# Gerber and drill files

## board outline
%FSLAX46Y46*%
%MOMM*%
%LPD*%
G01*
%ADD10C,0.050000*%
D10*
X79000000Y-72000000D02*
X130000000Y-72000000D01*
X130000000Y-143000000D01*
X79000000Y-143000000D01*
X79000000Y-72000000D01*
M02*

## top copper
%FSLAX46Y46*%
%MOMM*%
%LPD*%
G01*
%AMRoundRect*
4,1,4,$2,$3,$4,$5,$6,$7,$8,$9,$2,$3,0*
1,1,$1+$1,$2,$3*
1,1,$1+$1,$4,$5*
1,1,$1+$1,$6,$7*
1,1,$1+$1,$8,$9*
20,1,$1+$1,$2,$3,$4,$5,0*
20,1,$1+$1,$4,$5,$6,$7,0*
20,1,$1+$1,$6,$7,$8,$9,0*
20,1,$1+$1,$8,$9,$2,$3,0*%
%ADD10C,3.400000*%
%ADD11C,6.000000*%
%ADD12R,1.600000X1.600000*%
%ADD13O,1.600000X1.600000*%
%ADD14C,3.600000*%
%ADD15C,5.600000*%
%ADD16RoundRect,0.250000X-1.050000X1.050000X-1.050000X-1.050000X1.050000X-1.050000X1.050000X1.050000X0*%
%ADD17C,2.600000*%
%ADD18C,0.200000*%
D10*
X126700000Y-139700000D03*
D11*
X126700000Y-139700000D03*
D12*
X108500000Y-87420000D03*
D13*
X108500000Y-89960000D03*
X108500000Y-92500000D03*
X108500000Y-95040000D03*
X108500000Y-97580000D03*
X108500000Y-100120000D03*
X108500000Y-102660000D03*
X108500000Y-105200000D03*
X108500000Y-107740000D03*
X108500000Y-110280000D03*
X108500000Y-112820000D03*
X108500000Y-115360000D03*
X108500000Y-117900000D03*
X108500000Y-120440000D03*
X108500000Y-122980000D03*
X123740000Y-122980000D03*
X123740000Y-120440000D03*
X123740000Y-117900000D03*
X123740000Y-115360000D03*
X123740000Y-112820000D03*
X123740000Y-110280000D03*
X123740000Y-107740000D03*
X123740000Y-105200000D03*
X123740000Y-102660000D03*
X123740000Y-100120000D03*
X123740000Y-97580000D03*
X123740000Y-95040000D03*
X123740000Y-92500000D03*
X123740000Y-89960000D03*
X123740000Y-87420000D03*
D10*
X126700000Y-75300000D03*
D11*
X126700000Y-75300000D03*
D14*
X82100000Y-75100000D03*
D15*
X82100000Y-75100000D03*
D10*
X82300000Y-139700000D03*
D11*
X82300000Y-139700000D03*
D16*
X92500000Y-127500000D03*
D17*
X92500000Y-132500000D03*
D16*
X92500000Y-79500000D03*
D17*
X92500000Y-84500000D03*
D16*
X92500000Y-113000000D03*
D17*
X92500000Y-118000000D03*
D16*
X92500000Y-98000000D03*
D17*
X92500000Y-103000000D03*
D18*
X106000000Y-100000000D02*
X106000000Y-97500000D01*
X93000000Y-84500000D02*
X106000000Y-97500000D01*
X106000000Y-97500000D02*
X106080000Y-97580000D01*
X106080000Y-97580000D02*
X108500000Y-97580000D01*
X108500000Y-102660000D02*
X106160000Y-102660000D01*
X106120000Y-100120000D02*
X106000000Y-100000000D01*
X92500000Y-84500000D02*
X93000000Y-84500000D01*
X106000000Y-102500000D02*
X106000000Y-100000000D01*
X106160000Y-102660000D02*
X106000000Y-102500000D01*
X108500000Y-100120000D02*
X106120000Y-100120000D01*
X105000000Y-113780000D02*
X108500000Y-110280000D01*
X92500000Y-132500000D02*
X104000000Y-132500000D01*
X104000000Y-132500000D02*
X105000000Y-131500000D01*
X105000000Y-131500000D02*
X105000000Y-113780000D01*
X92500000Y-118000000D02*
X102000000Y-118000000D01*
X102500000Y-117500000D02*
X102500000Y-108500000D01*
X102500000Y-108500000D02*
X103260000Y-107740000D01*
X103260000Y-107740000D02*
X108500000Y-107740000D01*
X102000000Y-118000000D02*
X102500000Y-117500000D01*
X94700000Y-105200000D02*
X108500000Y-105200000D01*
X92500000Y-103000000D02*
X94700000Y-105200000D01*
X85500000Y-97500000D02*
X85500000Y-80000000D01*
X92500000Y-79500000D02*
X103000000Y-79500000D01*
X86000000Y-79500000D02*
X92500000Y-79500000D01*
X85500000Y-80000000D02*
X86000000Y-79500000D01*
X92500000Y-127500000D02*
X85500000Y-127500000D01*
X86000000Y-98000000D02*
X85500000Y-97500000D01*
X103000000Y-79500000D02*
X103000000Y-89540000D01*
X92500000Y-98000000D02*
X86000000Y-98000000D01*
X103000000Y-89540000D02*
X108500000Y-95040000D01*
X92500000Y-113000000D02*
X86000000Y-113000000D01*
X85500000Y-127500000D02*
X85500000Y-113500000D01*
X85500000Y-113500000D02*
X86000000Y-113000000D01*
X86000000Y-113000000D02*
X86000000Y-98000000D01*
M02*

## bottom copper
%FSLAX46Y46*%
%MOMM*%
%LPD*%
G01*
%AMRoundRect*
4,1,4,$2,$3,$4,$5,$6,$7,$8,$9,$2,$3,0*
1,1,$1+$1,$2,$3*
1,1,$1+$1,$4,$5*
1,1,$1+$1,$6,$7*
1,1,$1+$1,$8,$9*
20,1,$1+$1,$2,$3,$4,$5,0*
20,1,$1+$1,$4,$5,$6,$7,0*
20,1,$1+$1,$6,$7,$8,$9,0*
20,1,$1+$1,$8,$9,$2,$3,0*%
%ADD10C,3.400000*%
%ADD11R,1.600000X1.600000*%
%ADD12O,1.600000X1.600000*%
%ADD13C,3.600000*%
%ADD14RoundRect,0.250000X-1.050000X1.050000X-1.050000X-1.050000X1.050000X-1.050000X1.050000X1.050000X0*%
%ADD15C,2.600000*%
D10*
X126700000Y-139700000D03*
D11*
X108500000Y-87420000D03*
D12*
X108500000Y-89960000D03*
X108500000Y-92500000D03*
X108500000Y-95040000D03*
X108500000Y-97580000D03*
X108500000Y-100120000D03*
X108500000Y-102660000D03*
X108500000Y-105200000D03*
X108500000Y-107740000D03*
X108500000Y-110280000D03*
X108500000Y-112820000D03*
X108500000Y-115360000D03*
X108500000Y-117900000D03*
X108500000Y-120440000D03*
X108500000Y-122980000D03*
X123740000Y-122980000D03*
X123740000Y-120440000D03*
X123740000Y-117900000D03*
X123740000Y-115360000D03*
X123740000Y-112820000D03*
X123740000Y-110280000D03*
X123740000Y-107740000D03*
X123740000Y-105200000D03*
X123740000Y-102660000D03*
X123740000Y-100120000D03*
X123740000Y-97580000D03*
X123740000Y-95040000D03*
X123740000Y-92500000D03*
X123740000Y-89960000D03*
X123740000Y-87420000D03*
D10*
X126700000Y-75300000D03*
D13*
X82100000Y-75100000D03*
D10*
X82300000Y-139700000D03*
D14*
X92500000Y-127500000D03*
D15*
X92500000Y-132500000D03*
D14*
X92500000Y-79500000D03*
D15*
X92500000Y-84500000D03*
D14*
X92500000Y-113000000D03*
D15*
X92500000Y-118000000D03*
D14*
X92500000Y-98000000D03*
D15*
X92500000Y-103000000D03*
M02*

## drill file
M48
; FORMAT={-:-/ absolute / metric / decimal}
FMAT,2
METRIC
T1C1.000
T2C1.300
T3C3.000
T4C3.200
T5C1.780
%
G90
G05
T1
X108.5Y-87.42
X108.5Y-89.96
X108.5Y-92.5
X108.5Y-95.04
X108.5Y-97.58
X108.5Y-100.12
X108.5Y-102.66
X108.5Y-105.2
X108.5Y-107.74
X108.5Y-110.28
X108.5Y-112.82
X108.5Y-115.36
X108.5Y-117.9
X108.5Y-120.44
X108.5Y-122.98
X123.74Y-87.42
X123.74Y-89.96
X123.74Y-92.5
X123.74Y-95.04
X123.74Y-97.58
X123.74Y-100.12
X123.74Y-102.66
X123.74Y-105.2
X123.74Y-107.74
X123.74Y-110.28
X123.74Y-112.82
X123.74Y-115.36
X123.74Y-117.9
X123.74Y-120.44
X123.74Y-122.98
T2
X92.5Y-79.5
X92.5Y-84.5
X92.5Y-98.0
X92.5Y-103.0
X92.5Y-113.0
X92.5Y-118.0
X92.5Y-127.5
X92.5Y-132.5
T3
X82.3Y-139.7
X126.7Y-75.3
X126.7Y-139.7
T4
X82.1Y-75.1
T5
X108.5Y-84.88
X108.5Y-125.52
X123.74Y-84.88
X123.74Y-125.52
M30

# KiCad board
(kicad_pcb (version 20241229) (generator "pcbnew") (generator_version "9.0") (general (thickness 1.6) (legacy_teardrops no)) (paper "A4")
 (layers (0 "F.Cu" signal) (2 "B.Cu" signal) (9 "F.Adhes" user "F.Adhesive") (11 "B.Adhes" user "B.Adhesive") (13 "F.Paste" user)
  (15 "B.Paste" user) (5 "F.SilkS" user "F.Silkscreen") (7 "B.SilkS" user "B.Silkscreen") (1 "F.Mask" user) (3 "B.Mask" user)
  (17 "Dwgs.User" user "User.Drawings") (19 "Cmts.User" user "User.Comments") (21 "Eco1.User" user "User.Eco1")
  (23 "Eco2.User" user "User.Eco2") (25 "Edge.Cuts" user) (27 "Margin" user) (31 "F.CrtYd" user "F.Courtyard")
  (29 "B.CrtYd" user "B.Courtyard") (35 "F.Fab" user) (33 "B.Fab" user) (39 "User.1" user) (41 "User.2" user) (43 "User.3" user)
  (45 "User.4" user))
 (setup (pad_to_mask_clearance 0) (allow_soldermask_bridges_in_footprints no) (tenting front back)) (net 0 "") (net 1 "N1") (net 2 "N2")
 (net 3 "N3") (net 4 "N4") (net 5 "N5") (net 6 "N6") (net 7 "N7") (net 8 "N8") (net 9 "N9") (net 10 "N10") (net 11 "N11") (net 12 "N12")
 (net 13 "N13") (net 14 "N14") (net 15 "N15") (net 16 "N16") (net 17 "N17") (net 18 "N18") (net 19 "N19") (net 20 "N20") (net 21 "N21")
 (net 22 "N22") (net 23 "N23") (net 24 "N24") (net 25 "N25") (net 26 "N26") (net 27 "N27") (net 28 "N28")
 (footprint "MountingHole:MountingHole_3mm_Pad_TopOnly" (layer "F.Cu") (at 126.7 139.7)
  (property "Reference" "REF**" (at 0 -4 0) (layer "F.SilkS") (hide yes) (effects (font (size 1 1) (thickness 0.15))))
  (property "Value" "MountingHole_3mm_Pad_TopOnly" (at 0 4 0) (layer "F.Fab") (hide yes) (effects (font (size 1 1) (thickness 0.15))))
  (pad "1" thru_hole circle (at 0 0) (size 3.4 3.4) (drill 3) (layers "*.Cu" "*.Mask") (remove_unused_layers no))
  (pad "1" connect circle (at 0 0) (size 6 6) (layers "F.Cu" "F.Mask")))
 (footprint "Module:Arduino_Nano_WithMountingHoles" (layer "F.Cu") (at 108.5 87.42)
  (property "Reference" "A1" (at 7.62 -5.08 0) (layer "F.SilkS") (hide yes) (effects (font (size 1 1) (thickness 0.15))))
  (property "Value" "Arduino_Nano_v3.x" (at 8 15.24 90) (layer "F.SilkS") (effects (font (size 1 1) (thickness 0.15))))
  (pad "" np_thru_hole circle (at 0 -2.54) (size 1.78 1.78) (drill 1.78) (layers "*.Cu" "*.Mask"))
  (pad "" np_thru_hole circle (at 0 38.1) (size 1.78 1.78) (drill 1.78) (layers "*.Cu" "*.Mask"))
  (pad "" np_thru_hole circle (at 15.24 -2.54) (size 1.78 1.78) (drill 1.78) (layers "*.Cu" "*.Mask"))
  (pad "" np_thru_hole circle (at 15.24 38.1) (size 1.78 1.78) (drill 1.78) (layers "*.Cu" "*.Mask"))
  (pad "1" thru_hole rect (at 0 0) (size 1.6 1.6) (drill 1) (layers "*.Cu" "*.Mask") (remove_unused_layers no) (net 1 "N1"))
  (pad "2" thru_hole oval (at 0 2.54) (size 1.6 1.6) (drill 1) (layers "*.Cu" "*.Mask") (remove_unused_layers no) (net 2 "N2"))
  (pad "3" thru_hole oval (at 0 5.08) (size 1.6 1.6) (drill 1) (layers "*.Cu" "*.Mask") (remove_unused_layers no) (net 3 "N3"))
  (pad "4" thru_hole oval (at 0 7.62) (size 1.6 1.6) (drill 1) (layers "*.Cu" "*.Mask") (remove_unused_layers no) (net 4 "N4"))
  (pad "5" thru_hole oval (at 0 10.16) (size 1.6 1.6) (drill 1) (layers "*.Cu" "*.Mask") (remove_unused_layers no) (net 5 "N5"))
  (pad "6" thru_hole oval (at 0 12.7) (size 1.6 1.6) (drill 1) (layers "*.Cu" "*.Mask") (remove_unused_layers no) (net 5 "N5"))
  (pad "7" thru_hole oval (at 0 15.24) (size 1.6 1.6) (drill 1) (layers "*.Cu" "*.Mask") (remove_unused_layers no) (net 5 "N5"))
  (pad "8" thru_hole oval (at 0 17.78) (size 1.6 1.6) (drill 1) (layers "*.Cu" "*.Mask") (remove_unused_layers no) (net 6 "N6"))
  (pad "9" thru_hole oval (at 0 20.32) (size 1.6 1.6) (drill 1) (layers "*.Cu" "*.Mask") (remove_unused_layers no) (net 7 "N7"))
  (pad "10" thru_hole oval (at 0 22.86) (size 1.6 1.6) (drill 1) (layers "*.Cu" "*.Mask") (remove_unused_layers no) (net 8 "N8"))
  (pad "11" thru_hole oval (at 0 25.4) (size 1.6 1.6) (drill 1) (layers "*.Cu" "*.Mask") (remove_unused_layers no) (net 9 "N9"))
  (pad "12" thru_hole oval (at 0 27.94) (size 1.6 1.6) (drill 1) (layers "*.Cu" "*.Mask") (remove_unused_layers no) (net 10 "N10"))
  (pad "13" thru_hole oval (at 0 30.48) (size 1.6 1.6) (drill 1) (layers "*.Cu" "*.Mask") (remove_unused_layers no) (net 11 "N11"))
  (pad "14" thru_hole oval (at 0 33.02) (size 1.6 1.6) (drill 1) (layers "*.Cu" "*.Mask") (remove_unused_layers no) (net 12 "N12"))
  (pad "15" thru_hole oval (at 0 35.56) (size 1.6 1.6) (drill 1) (layers "*.Cu" "*.Mask") (remove_unused_layers no) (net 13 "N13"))
  (pad "16" thru_hole oval (at 15.24 35.56) (size 1.6 1.6) (drill 1) (layers "*.Cu" "*.Mask") (remove_unused_layers no) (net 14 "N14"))
  (pad "17" thru_hole oval (at 15.24 33.02) (size 1.6 1.6) (drill 1) (layers "*.Cu" "*.Mask") (remove_unused_layers no) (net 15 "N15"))
  (pad "18" thru_hole oval (at 15.24 30.48) (size 1.6 1.6) (drill 1) (layers "*.Cu" "*.Mask") (remove_unused_layers no) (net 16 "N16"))
  (pad "19" thru_hole oval (at 15.24 27.94) (size 1.6 1.6) (drill 1) (layers "*.Cu" "*.Mask") (remove_unused_layers no) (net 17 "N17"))
  (pad "20" thru_hole oval (at 15.24 25.4) (size 1.6 1.6) (drill 1) (layers "*.Cu" "*.Mask") (remove_unused_layers no) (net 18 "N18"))
  (pad "21" thru_hole oval (at 15.24 22.86) (size 1.6 1.6) (drill 1) (layers "*.Cu" "*.Mask") (remove_unused_layers no) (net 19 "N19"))
  (pad "22" thru_hole oval (at 15.24 20.32) (size 1.6 1.6) (drill 1) (layers "*.Cu" "*.Mask") (remove_unused_layers no) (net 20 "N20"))
  (pad "23" thru_hole oval (at 15.24 17.78) (size 1.6 1.6) (drill 1) (layers "*.Cu" "*.Mask") (remove_unused_layers no) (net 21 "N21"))
  (pad "24" thru_hole oval (at 15.24 15.24) (size 1.6 1.6) (drill 1) (layers "*.Cu" "*.Mask") (remove_unused_layers no) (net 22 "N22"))
  (pad "25" thru_hole oval (at 15.24 12.7) (size 1.6 1.6) (drill 1) (layers "*.Cu" "*.Mask") (remove_unused_layers no) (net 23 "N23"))
  (pad "26" thru_hole oval (at 15.24 10.16) (size 1.6 1.6) (drill 1) (layers "*.Cu" "*.Mask") (remove_unused_layers no) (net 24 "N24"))
  (pad "27" thru_hole oval (at 15.24 7.62) (size 1.6 1.6) (drill 1) (layers "*.Cu" "*.Mask") (remove_unused_layers no) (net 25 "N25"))
  (pad "28" thru_hole oval (at 15.24 5.08) (size 1.6 1.6) (drill 1) (layers "*.Cu" "*.Mask") (remove_unused_layers no) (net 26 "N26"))
  (pad "29" thru_hole oval (at 15.24 2.54) (size 1.6 1.6) (drill 1) (layers "*.Cu" "*.Mask") (remove_unused_layers no) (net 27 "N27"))
  (pad "30" thru_hole oval (at 15.24 0) (size 1.6 1.6) (drill 1) (layers "*.Cu" "*.Mask") (remove_unused_layers no) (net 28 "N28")))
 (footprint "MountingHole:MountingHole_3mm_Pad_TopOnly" (layer "F.Cu") (at 126.7 75.3)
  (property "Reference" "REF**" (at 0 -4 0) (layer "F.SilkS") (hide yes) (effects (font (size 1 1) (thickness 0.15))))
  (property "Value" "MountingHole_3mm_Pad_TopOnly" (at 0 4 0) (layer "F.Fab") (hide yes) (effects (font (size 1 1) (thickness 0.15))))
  (pad "1" thru_hole circle (at 0 0) (size 3.4 3.4) (drill 3) (layers "*.Cu" "*.Mask") (remove_unused_layers no))
  (pad "1" connect circle (at 0 0) (size 6 6) (layers "F.Cu" "F.Mask")))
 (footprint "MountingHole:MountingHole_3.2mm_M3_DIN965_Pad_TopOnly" (layer "F.Cu") (at 82.1 75.1)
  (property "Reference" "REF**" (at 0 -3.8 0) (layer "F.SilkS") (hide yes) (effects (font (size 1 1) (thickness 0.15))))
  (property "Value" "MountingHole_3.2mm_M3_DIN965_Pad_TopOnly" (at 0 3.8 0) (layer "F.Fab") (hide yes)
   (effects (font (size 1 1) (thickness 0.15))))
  (pad "1" thru_hole circle (at 0 0) (size 3.6 3.6) (drill 3.2) (layers "*.Cu" "*.Mask") (remove_unused_layers no))
  (pad "1" connect circle (at 0 0) (size 5.6 5.6) (layers "F.Cu" "F.Mask")))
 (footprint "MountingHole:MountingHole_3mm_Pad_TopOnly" (layer "F.Cu") (at 82.3 139.7)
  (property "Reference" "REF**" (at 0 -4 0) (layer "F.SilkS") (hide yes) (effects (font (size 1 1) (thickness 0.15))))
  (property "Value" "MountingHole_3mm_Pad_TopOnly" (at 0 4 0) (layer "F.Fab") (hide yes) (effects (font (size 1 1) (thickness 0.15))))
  (pad "1" thru_hole circle (at 0 0) (size 3.4 3.4) (drill 3) (layers "*.Cu" "*.Mask") (remove_unused_layers no))
  (pad "1" connect circle (at 0 0) (size 6 6) (layers "F.Cu" "F.Mask")))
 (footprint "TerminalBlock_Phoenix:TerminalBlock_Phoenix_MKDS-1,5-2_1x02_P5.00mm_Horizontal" (layer "F.Cu") (at 92.5 127.5 -90)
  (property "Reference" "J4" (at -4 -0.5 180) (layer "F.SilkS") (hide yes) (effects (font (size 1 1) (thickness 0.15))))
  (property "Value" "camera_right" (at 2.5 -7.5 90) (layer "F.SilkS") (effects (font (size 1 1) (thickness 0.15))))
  (pad "1" thru_hole roundrect (at 0 0 270) (size 2.6 2.6) (drill 1.3) (layers "*.Cu" "*.Mask") (remove_unused_layers no)
   (roundrect_rratio 0.096154) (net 4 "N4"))
  (pad "2" thru_hole circle (at 5 0 270) (size 2.6 2.6) (drill 1.3) (layers "*.Cu" "*.Mask") (remove_unused_layers no) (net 8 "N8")))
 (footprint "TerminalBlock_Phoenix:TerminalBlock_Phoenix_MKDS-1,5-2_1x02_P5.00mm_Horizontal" (layer "F.Cu") (at 92.5 79.5 -90)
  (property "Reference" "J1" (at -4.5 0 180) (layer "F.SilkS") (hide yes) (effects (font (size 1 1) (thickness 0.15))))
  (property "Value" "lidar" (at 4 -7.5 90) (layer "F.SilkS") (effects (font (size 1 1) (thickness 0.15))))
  (pad "1" thru_hole roundrect (at 0 0 270) (size 2.6 2.6) (drill 1.3) (layers "*.Cu" "*.Mask") (remove_unused_layers no)
   (roundrect_rratio 0.096154) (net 4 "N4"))
  (pad "2" thru_hole circle (at 5 0 270) (size 2.6 2.6) (drill 1.3) (layers "*.Cu" "*.Mask") (remove_unused_layers no) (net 5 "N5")))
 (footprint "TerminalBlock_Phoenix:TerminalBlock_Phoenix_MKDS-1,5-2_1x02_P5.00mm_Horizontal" (layer "F.Cu") (at 92.5 113 -90)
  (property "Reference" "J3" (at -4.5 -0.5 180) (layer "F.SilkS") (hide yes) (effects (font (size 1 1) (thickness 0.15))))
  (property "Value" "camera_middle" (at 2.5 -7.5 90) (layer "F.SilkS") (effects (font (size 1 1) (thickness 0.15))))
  (pad "1" thru_hole roundrect (at 0 0 270) (size 2.6 2.6) (drill 1.3) (layers "*.Cu" "*.Mask") (remove_unused_layers no)
   (roundrect_rratio 0.096154) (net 4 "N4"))
  (pad "2" thru_hole circle (at 5 0 270) (size 2.6 2.6) (drill 1.3) (layers "*.Cu" "*.Mask") (remove_unused_layers no) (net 7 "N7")))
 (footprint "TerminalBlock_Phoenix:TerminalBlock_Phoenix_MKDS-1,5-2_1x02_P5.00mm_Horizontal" (layer "F.Cu") (at 92.5 98 -90)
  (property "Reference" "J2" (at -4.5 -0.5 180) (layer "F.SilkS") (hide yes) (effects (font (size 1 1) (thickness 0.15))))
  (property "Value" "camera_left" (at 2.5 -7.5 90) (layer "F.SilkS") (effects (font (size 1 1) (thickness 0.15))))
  (pad "1" thru_hole roundrect (at 0 0 270) (size 2.6 2.6) (drill 1.3) (layers "*.Cu" "*.Mask") (remove_unused_layers no)
   (roundrect_rratio 0.096154) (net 4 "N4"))
  (pad "2" thru_hole circle (at 5 0 270) (size 2.6 2.6) (drill 1.3) (layers "*.Cu" "*.Mask") (remove_unused_layers no) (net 6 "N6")))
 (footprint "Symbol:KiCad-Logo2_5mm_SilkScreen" (layer "B.Cu") (at 114.75 78.1 180)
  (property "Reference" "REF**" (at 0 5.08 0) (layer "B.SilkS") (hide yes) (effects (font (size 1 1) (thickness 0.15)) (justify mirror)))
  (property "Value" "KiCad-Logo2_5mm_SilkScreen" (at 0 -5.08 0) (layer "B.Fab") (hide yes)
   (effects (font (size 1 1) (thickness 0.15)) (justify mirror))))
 (gr_rect (start 79 72) (end 130 143) (stroke (width 0.05) (type default)) (fill no) (layer "Edge.Cuts"))
 (segment (start 106 100) (end 106 97.5) (width 0.2) (layer "F.Cu") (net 5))
 (segment (start 93 84.5) (end 106 97.5) (width 0.2) (layer "F.Cu") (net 5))
 (segment (start 106 97.5) (end 106.08 97.58) (width 0.2) (layer "F.Cu") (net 5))
 (segment (start 106.08 97.58) (end 108.5 97.58) (width 0.2) (layer "F.Cu") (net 5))
 (segment (start 108.5 102.66) (end 106.16 102.66) (width 0.2) (layer "F.Cu") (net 5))
 (segment (start 106.12 100.12) (end 106 100) (width 0.2) (layer "F.Cu") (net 5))
 (segment (start 92.5 84.5) (end 93 84.5) (width 0.2) (layer "F.Cu") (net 5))
 (segment (start 106 102.5) (end 106 100) (width 0.2) (layer "F.Cu") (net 5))
 (segment (start 106.16 102.66) (end 106 102.5) (width 0.2) (layer "F.Cu") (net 5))
 (segment (start 108.5 100.12) (end 106.12 100.12) (width 0.2) (layer "F.Cu") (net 5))
 (segment (start 105 113.78) (end 108.5 110.28) (width 0.2) (layer "F.Cu") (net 8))
 (segment (start 92.5 132.5) (end 104 132.5) (width 0.2) (layer "F.Cu") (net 8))
 (segment (start 104 132.5) (end 105 131.5) (width 0.2) (layer "F.Cu") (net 8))
 (segment (start 105 131.5) (end 105 113.78) (width 0.2) (layer "F.Cu") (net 8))
 (segment (start 92.5 118) (end 102 118) (width 0.2) (layer "F.Cu") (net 7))
 (segment (start 102.5 117.5) (end 102.5 108.5) (width 0.2) (layer "F.Cu") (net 7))
 (segment (start 102.5 108.5) (end 103.26 107.74) (width 0.2) (layer "F.Cu") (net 7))
 (segment (start 103.26 107.74) (end 108.5 107.74) (width 0.2) (layer "F.Cu") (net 7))
 (segment (start 102 118) (end 102.5 117.5) (width 0.2) (layer "F.Cu") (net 7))
 (segment (start 94.7 105.2) (end 108.5 105.2) (width 0.2) (layer "F.Cu") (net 6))
 (segment (start 92.5 103) (end 94.7 105.2) (width 0.2) (layer "F.Cu") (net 6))
 (segment (start 85.5 97.5) (end 85.5 80) (width 0.2) (layer "F.Cu") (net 4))
 (segment (start 92.5 79.5) (end 103 79.5) (width 0.2) (layer "F.Cu") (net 4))
 (segment (start 86 79.5) (end 92.5 79.5) (width 0.2) (layer "F.Cu") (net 4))
 (segment (start 85.5 80) (end 86 79.5) (width 0.2) (layer "F.Cu") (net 4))
 (segment (start 92.5 127.5) (end 85.5 127.5) (width 0.2) (layer "F.Cu") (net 4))
 (segment (start 86 98) (end 85.5 97.5) (width 0.2) (layer "F.Cu") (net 4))
 (segment (start 103 79.5) (end 103 89.54) (width 0.2) (layer "F.Cu") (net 4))
 (segment (start 92.5 98) (end 86 98) (width 0.2) (layer "F.Cu") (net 4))
 (segment (start 103 89.54) (end 108.5 95.04) (width 0.2) (layer "F.Cu") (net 4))
 (segment (start 92.5 113) (end 86 113) (width 0.2) (layer "F.Cu") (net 4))
 (segment (start 85.5 127.5) (end 85.5 113.5) (width 0.2) (layer "F.Cu") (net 4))
 (segment (start 85.5 113.5) (end 86 113) (width 0.2) (layer "F.Cu") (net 4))
 (segment (start 86 113) (end 86 98) (width 0.2) (layer "F.Cu") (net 4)))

